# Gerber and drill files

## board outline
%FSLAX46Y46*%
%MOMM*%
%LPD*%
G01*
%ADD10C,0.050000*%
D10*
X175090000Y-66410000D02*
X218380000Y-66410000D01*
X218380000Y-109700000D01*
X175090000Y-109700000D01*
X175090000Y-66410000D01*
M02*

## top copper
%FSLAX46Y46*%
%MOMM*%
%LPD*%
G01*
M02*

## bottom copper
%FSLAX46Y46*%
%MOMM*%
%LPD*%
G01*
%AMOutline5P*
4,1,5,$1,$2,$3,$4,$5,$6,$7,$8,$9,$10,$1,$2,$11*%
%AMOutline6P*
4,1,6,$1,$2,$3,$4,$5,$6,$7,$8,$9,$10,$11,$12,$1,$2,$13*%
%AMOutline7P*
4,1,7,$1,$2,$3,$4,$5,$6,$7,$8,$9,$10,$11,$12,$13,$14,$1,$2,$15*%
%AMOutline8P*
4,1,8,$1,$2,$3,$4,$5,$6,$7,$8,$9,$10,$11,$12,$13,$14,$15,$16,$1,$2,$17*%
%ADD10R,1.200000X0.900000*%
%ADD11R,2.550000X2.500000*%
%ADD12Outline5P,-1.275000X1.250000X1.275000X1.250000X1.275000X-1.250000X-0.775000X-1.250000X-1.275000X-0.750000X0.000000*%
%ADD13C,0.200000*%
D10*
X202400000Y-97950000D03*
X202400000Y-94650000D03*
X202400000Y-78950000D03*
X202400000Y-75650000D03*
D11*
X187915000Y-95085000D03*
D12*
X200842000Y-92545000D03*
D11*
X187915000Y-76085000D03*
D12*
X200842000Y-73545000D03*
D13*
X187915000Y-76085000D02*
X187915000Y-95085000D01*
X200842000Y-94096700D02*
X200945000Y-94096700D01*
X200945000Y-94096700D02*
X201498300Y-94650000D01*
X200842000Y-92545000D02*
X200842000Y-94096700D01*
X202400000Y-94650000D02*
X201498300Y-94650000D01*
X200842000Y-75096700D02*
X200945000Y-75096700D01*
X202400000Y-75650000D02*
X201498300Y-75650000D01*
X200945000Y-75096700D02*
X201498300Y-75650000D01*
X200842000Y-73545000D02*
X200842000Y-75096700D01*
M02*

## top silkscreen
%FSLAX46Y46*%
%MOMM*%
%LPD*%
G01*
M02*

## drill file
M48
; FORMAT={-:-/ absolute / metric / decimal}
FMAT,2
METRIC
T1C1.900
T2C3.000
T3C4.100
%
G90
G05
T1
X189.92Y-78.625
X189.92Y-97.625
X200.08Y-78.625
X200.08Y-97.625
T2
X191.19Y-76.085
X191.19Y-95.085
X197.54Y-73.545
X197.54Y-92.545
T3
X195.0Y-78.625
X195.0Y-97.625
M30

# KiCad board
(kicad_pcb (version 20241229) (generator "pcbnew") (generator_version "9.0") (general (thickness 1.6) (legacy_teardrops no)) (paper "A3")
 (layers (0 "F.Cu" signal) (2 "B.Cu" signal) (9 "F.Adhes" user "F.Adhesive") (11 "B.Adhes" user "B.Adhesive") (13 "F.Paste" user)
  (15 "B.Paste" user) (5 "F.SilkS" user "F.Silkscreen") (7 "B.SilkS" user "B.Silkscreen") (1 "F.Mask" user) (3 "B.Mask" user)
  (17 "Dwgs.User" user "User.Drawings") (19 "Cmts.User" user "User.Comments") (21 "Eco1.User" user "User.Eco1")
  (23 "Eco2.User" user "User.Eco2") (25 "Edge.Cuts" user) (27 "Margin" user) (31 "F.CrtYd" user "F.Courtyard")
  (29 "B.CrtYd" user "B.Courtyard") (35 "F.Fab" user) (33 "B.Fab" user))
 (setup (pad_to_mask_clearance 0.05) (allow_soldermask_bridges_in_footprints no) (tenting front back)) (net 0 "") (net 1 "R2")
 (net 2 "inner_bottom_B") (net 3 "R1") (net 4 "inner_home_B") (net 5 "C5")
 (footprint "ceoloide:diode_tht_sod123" (layer "B.Cu") (at 202.4 96.3 90)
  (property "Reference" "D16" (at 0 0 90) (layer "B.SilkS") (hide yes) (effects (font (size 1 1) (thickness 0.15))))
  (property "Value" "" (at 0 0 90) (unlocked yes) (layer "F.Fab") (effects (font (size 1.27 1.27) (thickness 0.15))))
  (pad "1" smd rect (at -1.65 0 90) (size 0.9 1.2) (layers "B.Cu" "B.Mask" "B.Paste") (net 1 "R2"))
  (pad "2" smd rect (at 1.65 0 90) (size 0.9 1.2) (layers "B.Cu" "B.Mask" "B.Paste") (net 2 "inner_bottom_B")))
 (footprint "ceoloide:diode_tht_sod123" (layer "B.Cu") (at 202.4 77.3 90)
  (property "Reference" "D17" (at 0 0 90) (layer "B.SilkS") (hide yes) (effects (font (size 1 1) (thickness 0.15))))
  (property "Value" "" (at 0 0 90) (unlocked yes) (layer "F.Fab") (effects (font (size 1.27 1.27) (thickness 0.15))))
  (pad "1" smd rect (at -1.65 0 90) (size 0.9 1.2) (layers "B.Cu" "B.Mask" "B.Paste") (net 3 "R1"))
  (pad "2" smd rect (at 1.65 0 90) (size 0.9 1.2) (layers "B.Cu" "B.Mask" "B.Paste") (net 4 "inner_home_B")))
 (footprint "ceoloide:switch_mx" (layer "B.Cu") (at 195 97.625)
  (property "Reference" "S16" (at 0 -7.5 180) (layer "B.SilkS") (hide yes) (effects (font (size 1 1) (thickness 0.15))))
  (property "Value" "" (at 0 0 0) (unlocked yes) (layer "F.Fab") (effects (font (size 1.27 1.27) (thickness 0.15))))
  (pad "" np_thru_hole circle (at -5.08 0 180) (size 1.9 1.9) (drill 1.9) (layers "*.Cu" "*.Mask"))
  (pad "" np_thru_hole circle (at -3.81 -2.54 180) (size 3 3) (drill 3) (layers "*.Cu" "*.Mask"))
  (pad "" np_thru_hole circle (at 0 0 90) (size 4.1 4.1) (drill 4.1) (layers "*.Cu" "*.Mask"))
  (pad "" np_thru_hole circle (at 2.54 -5.08 180) (size 3 3) (drill 3) (layers "*.Cu" "*.Mask"))
  (pad "" np_thru_hole circle (at 5.08 0 180) (size 1.9 1.9) (drill 1.9) (layers "*.Cu" "*.Mask"))
  (pad "1" smd rect (at -7.085 -2.54) (size 2.55 2.5) (layers "B.Cu" "B.Mask" "B.Paste") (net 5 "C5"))
  (pad "2" smd roundrect (at 5.842 -5.08) (size 2.55 2.5) (layers "B.Cu" "B.Mask" "B.Paste") (roundrect_rratio 0) (chamfer_ratio 0.2)
   (chamfer bottom_left) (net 2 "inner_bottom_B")))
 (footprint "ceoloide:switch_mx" (layer "B.Cu") (at 195 78.625)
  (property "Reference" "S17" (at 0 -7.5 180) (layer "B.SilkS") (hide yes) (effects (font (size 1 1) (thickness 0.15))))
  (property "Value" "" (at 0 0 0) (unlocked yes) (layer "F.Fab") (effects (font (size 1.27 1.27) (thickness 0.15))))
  (pad "" np_thru_hole circle (at -5.08 0 180) (size 1.9 1.9) (drill 1.9) (layers "*.Cu" "*.Mask"))
  (pad "" np_thru_hole circle (at -3.81 -2.54 180) (size 3 3) (drill 3) (layers "*.Cu" "*.Mask"))
  (pad "" np_thru_hole circle (at 0 0 90) (size 4.1 4.1) (drill 4.1) (layers "*.Cu" "*.Mask"))
  (pad "" np_thru_hole circle (at 2.54 -5.08 180) (size 3 3) (drill 3) (layers "*.Cu" "*.Mask"))
  (pad "" np_thru_hole circle (at 5.08 0 180) (size 1.9 1.9) (drill 1.9) (layers "*.Cu" "*.Mask"))
  (pad "1" smd rect (at -7.085 -2.54) (size 2.55 2.5) (layers "B.Cu" "B.Mask" "B.Paste") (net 5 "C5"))
  (pad "2" smd roundrect (at 5.842 -5.08) (size 2.55 2.5) (layers "B.Cu" "B.Mask" "B.Paste") (roundrect_rratio 0) (chamfer_ratio 0.2)
   (chamfer bottom_left) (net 4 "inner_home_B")))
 (gr_rect (start 175.09 66.41) (end 218.38 109.7) (stroke (width 0.05) (type default)) (fill no) (layer "Edge.Cuts"))
 (segment (start 187.915 76.085) (end 187.915 95.085) (width 0.2) (layer "B.Cu") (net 5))
 (segment (start 200.842 94.0967) (end 200.945 94.0967) (width 0.2) (layer "B.Cu") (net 2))
 (segment (start 200.945 94.0967) (end 201.4983 94.65) (width 0.2) (layer "B.Cu") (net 2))
 (segment (start 200.842 92.545) (end 200.842 94.0967) (width 0.2) (layer "B.Cu") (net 2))
 (segment (start 202.4 94.65) (end 201.4983 94.65) (width 0.2) (layer "B.Cu") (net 2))
 (segment (start 200.842 75.0967) (end 200.945 75.0967) (width 0.2) (layer "B.Cu") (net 4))
 (segment (start 202.4 75.65) (end 201.4983 75.65) (width 0.2) (layer "B.Cu") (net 4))
 (segment (start 200.945 75.0967) (end 201.4983 75.65) (width 0.2) (layer "B.Cu") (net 4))
 (segment (start 200.842 73.545) (end 200.842 75.0967) (width 0.2) (layer "B.Cu") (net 4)))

